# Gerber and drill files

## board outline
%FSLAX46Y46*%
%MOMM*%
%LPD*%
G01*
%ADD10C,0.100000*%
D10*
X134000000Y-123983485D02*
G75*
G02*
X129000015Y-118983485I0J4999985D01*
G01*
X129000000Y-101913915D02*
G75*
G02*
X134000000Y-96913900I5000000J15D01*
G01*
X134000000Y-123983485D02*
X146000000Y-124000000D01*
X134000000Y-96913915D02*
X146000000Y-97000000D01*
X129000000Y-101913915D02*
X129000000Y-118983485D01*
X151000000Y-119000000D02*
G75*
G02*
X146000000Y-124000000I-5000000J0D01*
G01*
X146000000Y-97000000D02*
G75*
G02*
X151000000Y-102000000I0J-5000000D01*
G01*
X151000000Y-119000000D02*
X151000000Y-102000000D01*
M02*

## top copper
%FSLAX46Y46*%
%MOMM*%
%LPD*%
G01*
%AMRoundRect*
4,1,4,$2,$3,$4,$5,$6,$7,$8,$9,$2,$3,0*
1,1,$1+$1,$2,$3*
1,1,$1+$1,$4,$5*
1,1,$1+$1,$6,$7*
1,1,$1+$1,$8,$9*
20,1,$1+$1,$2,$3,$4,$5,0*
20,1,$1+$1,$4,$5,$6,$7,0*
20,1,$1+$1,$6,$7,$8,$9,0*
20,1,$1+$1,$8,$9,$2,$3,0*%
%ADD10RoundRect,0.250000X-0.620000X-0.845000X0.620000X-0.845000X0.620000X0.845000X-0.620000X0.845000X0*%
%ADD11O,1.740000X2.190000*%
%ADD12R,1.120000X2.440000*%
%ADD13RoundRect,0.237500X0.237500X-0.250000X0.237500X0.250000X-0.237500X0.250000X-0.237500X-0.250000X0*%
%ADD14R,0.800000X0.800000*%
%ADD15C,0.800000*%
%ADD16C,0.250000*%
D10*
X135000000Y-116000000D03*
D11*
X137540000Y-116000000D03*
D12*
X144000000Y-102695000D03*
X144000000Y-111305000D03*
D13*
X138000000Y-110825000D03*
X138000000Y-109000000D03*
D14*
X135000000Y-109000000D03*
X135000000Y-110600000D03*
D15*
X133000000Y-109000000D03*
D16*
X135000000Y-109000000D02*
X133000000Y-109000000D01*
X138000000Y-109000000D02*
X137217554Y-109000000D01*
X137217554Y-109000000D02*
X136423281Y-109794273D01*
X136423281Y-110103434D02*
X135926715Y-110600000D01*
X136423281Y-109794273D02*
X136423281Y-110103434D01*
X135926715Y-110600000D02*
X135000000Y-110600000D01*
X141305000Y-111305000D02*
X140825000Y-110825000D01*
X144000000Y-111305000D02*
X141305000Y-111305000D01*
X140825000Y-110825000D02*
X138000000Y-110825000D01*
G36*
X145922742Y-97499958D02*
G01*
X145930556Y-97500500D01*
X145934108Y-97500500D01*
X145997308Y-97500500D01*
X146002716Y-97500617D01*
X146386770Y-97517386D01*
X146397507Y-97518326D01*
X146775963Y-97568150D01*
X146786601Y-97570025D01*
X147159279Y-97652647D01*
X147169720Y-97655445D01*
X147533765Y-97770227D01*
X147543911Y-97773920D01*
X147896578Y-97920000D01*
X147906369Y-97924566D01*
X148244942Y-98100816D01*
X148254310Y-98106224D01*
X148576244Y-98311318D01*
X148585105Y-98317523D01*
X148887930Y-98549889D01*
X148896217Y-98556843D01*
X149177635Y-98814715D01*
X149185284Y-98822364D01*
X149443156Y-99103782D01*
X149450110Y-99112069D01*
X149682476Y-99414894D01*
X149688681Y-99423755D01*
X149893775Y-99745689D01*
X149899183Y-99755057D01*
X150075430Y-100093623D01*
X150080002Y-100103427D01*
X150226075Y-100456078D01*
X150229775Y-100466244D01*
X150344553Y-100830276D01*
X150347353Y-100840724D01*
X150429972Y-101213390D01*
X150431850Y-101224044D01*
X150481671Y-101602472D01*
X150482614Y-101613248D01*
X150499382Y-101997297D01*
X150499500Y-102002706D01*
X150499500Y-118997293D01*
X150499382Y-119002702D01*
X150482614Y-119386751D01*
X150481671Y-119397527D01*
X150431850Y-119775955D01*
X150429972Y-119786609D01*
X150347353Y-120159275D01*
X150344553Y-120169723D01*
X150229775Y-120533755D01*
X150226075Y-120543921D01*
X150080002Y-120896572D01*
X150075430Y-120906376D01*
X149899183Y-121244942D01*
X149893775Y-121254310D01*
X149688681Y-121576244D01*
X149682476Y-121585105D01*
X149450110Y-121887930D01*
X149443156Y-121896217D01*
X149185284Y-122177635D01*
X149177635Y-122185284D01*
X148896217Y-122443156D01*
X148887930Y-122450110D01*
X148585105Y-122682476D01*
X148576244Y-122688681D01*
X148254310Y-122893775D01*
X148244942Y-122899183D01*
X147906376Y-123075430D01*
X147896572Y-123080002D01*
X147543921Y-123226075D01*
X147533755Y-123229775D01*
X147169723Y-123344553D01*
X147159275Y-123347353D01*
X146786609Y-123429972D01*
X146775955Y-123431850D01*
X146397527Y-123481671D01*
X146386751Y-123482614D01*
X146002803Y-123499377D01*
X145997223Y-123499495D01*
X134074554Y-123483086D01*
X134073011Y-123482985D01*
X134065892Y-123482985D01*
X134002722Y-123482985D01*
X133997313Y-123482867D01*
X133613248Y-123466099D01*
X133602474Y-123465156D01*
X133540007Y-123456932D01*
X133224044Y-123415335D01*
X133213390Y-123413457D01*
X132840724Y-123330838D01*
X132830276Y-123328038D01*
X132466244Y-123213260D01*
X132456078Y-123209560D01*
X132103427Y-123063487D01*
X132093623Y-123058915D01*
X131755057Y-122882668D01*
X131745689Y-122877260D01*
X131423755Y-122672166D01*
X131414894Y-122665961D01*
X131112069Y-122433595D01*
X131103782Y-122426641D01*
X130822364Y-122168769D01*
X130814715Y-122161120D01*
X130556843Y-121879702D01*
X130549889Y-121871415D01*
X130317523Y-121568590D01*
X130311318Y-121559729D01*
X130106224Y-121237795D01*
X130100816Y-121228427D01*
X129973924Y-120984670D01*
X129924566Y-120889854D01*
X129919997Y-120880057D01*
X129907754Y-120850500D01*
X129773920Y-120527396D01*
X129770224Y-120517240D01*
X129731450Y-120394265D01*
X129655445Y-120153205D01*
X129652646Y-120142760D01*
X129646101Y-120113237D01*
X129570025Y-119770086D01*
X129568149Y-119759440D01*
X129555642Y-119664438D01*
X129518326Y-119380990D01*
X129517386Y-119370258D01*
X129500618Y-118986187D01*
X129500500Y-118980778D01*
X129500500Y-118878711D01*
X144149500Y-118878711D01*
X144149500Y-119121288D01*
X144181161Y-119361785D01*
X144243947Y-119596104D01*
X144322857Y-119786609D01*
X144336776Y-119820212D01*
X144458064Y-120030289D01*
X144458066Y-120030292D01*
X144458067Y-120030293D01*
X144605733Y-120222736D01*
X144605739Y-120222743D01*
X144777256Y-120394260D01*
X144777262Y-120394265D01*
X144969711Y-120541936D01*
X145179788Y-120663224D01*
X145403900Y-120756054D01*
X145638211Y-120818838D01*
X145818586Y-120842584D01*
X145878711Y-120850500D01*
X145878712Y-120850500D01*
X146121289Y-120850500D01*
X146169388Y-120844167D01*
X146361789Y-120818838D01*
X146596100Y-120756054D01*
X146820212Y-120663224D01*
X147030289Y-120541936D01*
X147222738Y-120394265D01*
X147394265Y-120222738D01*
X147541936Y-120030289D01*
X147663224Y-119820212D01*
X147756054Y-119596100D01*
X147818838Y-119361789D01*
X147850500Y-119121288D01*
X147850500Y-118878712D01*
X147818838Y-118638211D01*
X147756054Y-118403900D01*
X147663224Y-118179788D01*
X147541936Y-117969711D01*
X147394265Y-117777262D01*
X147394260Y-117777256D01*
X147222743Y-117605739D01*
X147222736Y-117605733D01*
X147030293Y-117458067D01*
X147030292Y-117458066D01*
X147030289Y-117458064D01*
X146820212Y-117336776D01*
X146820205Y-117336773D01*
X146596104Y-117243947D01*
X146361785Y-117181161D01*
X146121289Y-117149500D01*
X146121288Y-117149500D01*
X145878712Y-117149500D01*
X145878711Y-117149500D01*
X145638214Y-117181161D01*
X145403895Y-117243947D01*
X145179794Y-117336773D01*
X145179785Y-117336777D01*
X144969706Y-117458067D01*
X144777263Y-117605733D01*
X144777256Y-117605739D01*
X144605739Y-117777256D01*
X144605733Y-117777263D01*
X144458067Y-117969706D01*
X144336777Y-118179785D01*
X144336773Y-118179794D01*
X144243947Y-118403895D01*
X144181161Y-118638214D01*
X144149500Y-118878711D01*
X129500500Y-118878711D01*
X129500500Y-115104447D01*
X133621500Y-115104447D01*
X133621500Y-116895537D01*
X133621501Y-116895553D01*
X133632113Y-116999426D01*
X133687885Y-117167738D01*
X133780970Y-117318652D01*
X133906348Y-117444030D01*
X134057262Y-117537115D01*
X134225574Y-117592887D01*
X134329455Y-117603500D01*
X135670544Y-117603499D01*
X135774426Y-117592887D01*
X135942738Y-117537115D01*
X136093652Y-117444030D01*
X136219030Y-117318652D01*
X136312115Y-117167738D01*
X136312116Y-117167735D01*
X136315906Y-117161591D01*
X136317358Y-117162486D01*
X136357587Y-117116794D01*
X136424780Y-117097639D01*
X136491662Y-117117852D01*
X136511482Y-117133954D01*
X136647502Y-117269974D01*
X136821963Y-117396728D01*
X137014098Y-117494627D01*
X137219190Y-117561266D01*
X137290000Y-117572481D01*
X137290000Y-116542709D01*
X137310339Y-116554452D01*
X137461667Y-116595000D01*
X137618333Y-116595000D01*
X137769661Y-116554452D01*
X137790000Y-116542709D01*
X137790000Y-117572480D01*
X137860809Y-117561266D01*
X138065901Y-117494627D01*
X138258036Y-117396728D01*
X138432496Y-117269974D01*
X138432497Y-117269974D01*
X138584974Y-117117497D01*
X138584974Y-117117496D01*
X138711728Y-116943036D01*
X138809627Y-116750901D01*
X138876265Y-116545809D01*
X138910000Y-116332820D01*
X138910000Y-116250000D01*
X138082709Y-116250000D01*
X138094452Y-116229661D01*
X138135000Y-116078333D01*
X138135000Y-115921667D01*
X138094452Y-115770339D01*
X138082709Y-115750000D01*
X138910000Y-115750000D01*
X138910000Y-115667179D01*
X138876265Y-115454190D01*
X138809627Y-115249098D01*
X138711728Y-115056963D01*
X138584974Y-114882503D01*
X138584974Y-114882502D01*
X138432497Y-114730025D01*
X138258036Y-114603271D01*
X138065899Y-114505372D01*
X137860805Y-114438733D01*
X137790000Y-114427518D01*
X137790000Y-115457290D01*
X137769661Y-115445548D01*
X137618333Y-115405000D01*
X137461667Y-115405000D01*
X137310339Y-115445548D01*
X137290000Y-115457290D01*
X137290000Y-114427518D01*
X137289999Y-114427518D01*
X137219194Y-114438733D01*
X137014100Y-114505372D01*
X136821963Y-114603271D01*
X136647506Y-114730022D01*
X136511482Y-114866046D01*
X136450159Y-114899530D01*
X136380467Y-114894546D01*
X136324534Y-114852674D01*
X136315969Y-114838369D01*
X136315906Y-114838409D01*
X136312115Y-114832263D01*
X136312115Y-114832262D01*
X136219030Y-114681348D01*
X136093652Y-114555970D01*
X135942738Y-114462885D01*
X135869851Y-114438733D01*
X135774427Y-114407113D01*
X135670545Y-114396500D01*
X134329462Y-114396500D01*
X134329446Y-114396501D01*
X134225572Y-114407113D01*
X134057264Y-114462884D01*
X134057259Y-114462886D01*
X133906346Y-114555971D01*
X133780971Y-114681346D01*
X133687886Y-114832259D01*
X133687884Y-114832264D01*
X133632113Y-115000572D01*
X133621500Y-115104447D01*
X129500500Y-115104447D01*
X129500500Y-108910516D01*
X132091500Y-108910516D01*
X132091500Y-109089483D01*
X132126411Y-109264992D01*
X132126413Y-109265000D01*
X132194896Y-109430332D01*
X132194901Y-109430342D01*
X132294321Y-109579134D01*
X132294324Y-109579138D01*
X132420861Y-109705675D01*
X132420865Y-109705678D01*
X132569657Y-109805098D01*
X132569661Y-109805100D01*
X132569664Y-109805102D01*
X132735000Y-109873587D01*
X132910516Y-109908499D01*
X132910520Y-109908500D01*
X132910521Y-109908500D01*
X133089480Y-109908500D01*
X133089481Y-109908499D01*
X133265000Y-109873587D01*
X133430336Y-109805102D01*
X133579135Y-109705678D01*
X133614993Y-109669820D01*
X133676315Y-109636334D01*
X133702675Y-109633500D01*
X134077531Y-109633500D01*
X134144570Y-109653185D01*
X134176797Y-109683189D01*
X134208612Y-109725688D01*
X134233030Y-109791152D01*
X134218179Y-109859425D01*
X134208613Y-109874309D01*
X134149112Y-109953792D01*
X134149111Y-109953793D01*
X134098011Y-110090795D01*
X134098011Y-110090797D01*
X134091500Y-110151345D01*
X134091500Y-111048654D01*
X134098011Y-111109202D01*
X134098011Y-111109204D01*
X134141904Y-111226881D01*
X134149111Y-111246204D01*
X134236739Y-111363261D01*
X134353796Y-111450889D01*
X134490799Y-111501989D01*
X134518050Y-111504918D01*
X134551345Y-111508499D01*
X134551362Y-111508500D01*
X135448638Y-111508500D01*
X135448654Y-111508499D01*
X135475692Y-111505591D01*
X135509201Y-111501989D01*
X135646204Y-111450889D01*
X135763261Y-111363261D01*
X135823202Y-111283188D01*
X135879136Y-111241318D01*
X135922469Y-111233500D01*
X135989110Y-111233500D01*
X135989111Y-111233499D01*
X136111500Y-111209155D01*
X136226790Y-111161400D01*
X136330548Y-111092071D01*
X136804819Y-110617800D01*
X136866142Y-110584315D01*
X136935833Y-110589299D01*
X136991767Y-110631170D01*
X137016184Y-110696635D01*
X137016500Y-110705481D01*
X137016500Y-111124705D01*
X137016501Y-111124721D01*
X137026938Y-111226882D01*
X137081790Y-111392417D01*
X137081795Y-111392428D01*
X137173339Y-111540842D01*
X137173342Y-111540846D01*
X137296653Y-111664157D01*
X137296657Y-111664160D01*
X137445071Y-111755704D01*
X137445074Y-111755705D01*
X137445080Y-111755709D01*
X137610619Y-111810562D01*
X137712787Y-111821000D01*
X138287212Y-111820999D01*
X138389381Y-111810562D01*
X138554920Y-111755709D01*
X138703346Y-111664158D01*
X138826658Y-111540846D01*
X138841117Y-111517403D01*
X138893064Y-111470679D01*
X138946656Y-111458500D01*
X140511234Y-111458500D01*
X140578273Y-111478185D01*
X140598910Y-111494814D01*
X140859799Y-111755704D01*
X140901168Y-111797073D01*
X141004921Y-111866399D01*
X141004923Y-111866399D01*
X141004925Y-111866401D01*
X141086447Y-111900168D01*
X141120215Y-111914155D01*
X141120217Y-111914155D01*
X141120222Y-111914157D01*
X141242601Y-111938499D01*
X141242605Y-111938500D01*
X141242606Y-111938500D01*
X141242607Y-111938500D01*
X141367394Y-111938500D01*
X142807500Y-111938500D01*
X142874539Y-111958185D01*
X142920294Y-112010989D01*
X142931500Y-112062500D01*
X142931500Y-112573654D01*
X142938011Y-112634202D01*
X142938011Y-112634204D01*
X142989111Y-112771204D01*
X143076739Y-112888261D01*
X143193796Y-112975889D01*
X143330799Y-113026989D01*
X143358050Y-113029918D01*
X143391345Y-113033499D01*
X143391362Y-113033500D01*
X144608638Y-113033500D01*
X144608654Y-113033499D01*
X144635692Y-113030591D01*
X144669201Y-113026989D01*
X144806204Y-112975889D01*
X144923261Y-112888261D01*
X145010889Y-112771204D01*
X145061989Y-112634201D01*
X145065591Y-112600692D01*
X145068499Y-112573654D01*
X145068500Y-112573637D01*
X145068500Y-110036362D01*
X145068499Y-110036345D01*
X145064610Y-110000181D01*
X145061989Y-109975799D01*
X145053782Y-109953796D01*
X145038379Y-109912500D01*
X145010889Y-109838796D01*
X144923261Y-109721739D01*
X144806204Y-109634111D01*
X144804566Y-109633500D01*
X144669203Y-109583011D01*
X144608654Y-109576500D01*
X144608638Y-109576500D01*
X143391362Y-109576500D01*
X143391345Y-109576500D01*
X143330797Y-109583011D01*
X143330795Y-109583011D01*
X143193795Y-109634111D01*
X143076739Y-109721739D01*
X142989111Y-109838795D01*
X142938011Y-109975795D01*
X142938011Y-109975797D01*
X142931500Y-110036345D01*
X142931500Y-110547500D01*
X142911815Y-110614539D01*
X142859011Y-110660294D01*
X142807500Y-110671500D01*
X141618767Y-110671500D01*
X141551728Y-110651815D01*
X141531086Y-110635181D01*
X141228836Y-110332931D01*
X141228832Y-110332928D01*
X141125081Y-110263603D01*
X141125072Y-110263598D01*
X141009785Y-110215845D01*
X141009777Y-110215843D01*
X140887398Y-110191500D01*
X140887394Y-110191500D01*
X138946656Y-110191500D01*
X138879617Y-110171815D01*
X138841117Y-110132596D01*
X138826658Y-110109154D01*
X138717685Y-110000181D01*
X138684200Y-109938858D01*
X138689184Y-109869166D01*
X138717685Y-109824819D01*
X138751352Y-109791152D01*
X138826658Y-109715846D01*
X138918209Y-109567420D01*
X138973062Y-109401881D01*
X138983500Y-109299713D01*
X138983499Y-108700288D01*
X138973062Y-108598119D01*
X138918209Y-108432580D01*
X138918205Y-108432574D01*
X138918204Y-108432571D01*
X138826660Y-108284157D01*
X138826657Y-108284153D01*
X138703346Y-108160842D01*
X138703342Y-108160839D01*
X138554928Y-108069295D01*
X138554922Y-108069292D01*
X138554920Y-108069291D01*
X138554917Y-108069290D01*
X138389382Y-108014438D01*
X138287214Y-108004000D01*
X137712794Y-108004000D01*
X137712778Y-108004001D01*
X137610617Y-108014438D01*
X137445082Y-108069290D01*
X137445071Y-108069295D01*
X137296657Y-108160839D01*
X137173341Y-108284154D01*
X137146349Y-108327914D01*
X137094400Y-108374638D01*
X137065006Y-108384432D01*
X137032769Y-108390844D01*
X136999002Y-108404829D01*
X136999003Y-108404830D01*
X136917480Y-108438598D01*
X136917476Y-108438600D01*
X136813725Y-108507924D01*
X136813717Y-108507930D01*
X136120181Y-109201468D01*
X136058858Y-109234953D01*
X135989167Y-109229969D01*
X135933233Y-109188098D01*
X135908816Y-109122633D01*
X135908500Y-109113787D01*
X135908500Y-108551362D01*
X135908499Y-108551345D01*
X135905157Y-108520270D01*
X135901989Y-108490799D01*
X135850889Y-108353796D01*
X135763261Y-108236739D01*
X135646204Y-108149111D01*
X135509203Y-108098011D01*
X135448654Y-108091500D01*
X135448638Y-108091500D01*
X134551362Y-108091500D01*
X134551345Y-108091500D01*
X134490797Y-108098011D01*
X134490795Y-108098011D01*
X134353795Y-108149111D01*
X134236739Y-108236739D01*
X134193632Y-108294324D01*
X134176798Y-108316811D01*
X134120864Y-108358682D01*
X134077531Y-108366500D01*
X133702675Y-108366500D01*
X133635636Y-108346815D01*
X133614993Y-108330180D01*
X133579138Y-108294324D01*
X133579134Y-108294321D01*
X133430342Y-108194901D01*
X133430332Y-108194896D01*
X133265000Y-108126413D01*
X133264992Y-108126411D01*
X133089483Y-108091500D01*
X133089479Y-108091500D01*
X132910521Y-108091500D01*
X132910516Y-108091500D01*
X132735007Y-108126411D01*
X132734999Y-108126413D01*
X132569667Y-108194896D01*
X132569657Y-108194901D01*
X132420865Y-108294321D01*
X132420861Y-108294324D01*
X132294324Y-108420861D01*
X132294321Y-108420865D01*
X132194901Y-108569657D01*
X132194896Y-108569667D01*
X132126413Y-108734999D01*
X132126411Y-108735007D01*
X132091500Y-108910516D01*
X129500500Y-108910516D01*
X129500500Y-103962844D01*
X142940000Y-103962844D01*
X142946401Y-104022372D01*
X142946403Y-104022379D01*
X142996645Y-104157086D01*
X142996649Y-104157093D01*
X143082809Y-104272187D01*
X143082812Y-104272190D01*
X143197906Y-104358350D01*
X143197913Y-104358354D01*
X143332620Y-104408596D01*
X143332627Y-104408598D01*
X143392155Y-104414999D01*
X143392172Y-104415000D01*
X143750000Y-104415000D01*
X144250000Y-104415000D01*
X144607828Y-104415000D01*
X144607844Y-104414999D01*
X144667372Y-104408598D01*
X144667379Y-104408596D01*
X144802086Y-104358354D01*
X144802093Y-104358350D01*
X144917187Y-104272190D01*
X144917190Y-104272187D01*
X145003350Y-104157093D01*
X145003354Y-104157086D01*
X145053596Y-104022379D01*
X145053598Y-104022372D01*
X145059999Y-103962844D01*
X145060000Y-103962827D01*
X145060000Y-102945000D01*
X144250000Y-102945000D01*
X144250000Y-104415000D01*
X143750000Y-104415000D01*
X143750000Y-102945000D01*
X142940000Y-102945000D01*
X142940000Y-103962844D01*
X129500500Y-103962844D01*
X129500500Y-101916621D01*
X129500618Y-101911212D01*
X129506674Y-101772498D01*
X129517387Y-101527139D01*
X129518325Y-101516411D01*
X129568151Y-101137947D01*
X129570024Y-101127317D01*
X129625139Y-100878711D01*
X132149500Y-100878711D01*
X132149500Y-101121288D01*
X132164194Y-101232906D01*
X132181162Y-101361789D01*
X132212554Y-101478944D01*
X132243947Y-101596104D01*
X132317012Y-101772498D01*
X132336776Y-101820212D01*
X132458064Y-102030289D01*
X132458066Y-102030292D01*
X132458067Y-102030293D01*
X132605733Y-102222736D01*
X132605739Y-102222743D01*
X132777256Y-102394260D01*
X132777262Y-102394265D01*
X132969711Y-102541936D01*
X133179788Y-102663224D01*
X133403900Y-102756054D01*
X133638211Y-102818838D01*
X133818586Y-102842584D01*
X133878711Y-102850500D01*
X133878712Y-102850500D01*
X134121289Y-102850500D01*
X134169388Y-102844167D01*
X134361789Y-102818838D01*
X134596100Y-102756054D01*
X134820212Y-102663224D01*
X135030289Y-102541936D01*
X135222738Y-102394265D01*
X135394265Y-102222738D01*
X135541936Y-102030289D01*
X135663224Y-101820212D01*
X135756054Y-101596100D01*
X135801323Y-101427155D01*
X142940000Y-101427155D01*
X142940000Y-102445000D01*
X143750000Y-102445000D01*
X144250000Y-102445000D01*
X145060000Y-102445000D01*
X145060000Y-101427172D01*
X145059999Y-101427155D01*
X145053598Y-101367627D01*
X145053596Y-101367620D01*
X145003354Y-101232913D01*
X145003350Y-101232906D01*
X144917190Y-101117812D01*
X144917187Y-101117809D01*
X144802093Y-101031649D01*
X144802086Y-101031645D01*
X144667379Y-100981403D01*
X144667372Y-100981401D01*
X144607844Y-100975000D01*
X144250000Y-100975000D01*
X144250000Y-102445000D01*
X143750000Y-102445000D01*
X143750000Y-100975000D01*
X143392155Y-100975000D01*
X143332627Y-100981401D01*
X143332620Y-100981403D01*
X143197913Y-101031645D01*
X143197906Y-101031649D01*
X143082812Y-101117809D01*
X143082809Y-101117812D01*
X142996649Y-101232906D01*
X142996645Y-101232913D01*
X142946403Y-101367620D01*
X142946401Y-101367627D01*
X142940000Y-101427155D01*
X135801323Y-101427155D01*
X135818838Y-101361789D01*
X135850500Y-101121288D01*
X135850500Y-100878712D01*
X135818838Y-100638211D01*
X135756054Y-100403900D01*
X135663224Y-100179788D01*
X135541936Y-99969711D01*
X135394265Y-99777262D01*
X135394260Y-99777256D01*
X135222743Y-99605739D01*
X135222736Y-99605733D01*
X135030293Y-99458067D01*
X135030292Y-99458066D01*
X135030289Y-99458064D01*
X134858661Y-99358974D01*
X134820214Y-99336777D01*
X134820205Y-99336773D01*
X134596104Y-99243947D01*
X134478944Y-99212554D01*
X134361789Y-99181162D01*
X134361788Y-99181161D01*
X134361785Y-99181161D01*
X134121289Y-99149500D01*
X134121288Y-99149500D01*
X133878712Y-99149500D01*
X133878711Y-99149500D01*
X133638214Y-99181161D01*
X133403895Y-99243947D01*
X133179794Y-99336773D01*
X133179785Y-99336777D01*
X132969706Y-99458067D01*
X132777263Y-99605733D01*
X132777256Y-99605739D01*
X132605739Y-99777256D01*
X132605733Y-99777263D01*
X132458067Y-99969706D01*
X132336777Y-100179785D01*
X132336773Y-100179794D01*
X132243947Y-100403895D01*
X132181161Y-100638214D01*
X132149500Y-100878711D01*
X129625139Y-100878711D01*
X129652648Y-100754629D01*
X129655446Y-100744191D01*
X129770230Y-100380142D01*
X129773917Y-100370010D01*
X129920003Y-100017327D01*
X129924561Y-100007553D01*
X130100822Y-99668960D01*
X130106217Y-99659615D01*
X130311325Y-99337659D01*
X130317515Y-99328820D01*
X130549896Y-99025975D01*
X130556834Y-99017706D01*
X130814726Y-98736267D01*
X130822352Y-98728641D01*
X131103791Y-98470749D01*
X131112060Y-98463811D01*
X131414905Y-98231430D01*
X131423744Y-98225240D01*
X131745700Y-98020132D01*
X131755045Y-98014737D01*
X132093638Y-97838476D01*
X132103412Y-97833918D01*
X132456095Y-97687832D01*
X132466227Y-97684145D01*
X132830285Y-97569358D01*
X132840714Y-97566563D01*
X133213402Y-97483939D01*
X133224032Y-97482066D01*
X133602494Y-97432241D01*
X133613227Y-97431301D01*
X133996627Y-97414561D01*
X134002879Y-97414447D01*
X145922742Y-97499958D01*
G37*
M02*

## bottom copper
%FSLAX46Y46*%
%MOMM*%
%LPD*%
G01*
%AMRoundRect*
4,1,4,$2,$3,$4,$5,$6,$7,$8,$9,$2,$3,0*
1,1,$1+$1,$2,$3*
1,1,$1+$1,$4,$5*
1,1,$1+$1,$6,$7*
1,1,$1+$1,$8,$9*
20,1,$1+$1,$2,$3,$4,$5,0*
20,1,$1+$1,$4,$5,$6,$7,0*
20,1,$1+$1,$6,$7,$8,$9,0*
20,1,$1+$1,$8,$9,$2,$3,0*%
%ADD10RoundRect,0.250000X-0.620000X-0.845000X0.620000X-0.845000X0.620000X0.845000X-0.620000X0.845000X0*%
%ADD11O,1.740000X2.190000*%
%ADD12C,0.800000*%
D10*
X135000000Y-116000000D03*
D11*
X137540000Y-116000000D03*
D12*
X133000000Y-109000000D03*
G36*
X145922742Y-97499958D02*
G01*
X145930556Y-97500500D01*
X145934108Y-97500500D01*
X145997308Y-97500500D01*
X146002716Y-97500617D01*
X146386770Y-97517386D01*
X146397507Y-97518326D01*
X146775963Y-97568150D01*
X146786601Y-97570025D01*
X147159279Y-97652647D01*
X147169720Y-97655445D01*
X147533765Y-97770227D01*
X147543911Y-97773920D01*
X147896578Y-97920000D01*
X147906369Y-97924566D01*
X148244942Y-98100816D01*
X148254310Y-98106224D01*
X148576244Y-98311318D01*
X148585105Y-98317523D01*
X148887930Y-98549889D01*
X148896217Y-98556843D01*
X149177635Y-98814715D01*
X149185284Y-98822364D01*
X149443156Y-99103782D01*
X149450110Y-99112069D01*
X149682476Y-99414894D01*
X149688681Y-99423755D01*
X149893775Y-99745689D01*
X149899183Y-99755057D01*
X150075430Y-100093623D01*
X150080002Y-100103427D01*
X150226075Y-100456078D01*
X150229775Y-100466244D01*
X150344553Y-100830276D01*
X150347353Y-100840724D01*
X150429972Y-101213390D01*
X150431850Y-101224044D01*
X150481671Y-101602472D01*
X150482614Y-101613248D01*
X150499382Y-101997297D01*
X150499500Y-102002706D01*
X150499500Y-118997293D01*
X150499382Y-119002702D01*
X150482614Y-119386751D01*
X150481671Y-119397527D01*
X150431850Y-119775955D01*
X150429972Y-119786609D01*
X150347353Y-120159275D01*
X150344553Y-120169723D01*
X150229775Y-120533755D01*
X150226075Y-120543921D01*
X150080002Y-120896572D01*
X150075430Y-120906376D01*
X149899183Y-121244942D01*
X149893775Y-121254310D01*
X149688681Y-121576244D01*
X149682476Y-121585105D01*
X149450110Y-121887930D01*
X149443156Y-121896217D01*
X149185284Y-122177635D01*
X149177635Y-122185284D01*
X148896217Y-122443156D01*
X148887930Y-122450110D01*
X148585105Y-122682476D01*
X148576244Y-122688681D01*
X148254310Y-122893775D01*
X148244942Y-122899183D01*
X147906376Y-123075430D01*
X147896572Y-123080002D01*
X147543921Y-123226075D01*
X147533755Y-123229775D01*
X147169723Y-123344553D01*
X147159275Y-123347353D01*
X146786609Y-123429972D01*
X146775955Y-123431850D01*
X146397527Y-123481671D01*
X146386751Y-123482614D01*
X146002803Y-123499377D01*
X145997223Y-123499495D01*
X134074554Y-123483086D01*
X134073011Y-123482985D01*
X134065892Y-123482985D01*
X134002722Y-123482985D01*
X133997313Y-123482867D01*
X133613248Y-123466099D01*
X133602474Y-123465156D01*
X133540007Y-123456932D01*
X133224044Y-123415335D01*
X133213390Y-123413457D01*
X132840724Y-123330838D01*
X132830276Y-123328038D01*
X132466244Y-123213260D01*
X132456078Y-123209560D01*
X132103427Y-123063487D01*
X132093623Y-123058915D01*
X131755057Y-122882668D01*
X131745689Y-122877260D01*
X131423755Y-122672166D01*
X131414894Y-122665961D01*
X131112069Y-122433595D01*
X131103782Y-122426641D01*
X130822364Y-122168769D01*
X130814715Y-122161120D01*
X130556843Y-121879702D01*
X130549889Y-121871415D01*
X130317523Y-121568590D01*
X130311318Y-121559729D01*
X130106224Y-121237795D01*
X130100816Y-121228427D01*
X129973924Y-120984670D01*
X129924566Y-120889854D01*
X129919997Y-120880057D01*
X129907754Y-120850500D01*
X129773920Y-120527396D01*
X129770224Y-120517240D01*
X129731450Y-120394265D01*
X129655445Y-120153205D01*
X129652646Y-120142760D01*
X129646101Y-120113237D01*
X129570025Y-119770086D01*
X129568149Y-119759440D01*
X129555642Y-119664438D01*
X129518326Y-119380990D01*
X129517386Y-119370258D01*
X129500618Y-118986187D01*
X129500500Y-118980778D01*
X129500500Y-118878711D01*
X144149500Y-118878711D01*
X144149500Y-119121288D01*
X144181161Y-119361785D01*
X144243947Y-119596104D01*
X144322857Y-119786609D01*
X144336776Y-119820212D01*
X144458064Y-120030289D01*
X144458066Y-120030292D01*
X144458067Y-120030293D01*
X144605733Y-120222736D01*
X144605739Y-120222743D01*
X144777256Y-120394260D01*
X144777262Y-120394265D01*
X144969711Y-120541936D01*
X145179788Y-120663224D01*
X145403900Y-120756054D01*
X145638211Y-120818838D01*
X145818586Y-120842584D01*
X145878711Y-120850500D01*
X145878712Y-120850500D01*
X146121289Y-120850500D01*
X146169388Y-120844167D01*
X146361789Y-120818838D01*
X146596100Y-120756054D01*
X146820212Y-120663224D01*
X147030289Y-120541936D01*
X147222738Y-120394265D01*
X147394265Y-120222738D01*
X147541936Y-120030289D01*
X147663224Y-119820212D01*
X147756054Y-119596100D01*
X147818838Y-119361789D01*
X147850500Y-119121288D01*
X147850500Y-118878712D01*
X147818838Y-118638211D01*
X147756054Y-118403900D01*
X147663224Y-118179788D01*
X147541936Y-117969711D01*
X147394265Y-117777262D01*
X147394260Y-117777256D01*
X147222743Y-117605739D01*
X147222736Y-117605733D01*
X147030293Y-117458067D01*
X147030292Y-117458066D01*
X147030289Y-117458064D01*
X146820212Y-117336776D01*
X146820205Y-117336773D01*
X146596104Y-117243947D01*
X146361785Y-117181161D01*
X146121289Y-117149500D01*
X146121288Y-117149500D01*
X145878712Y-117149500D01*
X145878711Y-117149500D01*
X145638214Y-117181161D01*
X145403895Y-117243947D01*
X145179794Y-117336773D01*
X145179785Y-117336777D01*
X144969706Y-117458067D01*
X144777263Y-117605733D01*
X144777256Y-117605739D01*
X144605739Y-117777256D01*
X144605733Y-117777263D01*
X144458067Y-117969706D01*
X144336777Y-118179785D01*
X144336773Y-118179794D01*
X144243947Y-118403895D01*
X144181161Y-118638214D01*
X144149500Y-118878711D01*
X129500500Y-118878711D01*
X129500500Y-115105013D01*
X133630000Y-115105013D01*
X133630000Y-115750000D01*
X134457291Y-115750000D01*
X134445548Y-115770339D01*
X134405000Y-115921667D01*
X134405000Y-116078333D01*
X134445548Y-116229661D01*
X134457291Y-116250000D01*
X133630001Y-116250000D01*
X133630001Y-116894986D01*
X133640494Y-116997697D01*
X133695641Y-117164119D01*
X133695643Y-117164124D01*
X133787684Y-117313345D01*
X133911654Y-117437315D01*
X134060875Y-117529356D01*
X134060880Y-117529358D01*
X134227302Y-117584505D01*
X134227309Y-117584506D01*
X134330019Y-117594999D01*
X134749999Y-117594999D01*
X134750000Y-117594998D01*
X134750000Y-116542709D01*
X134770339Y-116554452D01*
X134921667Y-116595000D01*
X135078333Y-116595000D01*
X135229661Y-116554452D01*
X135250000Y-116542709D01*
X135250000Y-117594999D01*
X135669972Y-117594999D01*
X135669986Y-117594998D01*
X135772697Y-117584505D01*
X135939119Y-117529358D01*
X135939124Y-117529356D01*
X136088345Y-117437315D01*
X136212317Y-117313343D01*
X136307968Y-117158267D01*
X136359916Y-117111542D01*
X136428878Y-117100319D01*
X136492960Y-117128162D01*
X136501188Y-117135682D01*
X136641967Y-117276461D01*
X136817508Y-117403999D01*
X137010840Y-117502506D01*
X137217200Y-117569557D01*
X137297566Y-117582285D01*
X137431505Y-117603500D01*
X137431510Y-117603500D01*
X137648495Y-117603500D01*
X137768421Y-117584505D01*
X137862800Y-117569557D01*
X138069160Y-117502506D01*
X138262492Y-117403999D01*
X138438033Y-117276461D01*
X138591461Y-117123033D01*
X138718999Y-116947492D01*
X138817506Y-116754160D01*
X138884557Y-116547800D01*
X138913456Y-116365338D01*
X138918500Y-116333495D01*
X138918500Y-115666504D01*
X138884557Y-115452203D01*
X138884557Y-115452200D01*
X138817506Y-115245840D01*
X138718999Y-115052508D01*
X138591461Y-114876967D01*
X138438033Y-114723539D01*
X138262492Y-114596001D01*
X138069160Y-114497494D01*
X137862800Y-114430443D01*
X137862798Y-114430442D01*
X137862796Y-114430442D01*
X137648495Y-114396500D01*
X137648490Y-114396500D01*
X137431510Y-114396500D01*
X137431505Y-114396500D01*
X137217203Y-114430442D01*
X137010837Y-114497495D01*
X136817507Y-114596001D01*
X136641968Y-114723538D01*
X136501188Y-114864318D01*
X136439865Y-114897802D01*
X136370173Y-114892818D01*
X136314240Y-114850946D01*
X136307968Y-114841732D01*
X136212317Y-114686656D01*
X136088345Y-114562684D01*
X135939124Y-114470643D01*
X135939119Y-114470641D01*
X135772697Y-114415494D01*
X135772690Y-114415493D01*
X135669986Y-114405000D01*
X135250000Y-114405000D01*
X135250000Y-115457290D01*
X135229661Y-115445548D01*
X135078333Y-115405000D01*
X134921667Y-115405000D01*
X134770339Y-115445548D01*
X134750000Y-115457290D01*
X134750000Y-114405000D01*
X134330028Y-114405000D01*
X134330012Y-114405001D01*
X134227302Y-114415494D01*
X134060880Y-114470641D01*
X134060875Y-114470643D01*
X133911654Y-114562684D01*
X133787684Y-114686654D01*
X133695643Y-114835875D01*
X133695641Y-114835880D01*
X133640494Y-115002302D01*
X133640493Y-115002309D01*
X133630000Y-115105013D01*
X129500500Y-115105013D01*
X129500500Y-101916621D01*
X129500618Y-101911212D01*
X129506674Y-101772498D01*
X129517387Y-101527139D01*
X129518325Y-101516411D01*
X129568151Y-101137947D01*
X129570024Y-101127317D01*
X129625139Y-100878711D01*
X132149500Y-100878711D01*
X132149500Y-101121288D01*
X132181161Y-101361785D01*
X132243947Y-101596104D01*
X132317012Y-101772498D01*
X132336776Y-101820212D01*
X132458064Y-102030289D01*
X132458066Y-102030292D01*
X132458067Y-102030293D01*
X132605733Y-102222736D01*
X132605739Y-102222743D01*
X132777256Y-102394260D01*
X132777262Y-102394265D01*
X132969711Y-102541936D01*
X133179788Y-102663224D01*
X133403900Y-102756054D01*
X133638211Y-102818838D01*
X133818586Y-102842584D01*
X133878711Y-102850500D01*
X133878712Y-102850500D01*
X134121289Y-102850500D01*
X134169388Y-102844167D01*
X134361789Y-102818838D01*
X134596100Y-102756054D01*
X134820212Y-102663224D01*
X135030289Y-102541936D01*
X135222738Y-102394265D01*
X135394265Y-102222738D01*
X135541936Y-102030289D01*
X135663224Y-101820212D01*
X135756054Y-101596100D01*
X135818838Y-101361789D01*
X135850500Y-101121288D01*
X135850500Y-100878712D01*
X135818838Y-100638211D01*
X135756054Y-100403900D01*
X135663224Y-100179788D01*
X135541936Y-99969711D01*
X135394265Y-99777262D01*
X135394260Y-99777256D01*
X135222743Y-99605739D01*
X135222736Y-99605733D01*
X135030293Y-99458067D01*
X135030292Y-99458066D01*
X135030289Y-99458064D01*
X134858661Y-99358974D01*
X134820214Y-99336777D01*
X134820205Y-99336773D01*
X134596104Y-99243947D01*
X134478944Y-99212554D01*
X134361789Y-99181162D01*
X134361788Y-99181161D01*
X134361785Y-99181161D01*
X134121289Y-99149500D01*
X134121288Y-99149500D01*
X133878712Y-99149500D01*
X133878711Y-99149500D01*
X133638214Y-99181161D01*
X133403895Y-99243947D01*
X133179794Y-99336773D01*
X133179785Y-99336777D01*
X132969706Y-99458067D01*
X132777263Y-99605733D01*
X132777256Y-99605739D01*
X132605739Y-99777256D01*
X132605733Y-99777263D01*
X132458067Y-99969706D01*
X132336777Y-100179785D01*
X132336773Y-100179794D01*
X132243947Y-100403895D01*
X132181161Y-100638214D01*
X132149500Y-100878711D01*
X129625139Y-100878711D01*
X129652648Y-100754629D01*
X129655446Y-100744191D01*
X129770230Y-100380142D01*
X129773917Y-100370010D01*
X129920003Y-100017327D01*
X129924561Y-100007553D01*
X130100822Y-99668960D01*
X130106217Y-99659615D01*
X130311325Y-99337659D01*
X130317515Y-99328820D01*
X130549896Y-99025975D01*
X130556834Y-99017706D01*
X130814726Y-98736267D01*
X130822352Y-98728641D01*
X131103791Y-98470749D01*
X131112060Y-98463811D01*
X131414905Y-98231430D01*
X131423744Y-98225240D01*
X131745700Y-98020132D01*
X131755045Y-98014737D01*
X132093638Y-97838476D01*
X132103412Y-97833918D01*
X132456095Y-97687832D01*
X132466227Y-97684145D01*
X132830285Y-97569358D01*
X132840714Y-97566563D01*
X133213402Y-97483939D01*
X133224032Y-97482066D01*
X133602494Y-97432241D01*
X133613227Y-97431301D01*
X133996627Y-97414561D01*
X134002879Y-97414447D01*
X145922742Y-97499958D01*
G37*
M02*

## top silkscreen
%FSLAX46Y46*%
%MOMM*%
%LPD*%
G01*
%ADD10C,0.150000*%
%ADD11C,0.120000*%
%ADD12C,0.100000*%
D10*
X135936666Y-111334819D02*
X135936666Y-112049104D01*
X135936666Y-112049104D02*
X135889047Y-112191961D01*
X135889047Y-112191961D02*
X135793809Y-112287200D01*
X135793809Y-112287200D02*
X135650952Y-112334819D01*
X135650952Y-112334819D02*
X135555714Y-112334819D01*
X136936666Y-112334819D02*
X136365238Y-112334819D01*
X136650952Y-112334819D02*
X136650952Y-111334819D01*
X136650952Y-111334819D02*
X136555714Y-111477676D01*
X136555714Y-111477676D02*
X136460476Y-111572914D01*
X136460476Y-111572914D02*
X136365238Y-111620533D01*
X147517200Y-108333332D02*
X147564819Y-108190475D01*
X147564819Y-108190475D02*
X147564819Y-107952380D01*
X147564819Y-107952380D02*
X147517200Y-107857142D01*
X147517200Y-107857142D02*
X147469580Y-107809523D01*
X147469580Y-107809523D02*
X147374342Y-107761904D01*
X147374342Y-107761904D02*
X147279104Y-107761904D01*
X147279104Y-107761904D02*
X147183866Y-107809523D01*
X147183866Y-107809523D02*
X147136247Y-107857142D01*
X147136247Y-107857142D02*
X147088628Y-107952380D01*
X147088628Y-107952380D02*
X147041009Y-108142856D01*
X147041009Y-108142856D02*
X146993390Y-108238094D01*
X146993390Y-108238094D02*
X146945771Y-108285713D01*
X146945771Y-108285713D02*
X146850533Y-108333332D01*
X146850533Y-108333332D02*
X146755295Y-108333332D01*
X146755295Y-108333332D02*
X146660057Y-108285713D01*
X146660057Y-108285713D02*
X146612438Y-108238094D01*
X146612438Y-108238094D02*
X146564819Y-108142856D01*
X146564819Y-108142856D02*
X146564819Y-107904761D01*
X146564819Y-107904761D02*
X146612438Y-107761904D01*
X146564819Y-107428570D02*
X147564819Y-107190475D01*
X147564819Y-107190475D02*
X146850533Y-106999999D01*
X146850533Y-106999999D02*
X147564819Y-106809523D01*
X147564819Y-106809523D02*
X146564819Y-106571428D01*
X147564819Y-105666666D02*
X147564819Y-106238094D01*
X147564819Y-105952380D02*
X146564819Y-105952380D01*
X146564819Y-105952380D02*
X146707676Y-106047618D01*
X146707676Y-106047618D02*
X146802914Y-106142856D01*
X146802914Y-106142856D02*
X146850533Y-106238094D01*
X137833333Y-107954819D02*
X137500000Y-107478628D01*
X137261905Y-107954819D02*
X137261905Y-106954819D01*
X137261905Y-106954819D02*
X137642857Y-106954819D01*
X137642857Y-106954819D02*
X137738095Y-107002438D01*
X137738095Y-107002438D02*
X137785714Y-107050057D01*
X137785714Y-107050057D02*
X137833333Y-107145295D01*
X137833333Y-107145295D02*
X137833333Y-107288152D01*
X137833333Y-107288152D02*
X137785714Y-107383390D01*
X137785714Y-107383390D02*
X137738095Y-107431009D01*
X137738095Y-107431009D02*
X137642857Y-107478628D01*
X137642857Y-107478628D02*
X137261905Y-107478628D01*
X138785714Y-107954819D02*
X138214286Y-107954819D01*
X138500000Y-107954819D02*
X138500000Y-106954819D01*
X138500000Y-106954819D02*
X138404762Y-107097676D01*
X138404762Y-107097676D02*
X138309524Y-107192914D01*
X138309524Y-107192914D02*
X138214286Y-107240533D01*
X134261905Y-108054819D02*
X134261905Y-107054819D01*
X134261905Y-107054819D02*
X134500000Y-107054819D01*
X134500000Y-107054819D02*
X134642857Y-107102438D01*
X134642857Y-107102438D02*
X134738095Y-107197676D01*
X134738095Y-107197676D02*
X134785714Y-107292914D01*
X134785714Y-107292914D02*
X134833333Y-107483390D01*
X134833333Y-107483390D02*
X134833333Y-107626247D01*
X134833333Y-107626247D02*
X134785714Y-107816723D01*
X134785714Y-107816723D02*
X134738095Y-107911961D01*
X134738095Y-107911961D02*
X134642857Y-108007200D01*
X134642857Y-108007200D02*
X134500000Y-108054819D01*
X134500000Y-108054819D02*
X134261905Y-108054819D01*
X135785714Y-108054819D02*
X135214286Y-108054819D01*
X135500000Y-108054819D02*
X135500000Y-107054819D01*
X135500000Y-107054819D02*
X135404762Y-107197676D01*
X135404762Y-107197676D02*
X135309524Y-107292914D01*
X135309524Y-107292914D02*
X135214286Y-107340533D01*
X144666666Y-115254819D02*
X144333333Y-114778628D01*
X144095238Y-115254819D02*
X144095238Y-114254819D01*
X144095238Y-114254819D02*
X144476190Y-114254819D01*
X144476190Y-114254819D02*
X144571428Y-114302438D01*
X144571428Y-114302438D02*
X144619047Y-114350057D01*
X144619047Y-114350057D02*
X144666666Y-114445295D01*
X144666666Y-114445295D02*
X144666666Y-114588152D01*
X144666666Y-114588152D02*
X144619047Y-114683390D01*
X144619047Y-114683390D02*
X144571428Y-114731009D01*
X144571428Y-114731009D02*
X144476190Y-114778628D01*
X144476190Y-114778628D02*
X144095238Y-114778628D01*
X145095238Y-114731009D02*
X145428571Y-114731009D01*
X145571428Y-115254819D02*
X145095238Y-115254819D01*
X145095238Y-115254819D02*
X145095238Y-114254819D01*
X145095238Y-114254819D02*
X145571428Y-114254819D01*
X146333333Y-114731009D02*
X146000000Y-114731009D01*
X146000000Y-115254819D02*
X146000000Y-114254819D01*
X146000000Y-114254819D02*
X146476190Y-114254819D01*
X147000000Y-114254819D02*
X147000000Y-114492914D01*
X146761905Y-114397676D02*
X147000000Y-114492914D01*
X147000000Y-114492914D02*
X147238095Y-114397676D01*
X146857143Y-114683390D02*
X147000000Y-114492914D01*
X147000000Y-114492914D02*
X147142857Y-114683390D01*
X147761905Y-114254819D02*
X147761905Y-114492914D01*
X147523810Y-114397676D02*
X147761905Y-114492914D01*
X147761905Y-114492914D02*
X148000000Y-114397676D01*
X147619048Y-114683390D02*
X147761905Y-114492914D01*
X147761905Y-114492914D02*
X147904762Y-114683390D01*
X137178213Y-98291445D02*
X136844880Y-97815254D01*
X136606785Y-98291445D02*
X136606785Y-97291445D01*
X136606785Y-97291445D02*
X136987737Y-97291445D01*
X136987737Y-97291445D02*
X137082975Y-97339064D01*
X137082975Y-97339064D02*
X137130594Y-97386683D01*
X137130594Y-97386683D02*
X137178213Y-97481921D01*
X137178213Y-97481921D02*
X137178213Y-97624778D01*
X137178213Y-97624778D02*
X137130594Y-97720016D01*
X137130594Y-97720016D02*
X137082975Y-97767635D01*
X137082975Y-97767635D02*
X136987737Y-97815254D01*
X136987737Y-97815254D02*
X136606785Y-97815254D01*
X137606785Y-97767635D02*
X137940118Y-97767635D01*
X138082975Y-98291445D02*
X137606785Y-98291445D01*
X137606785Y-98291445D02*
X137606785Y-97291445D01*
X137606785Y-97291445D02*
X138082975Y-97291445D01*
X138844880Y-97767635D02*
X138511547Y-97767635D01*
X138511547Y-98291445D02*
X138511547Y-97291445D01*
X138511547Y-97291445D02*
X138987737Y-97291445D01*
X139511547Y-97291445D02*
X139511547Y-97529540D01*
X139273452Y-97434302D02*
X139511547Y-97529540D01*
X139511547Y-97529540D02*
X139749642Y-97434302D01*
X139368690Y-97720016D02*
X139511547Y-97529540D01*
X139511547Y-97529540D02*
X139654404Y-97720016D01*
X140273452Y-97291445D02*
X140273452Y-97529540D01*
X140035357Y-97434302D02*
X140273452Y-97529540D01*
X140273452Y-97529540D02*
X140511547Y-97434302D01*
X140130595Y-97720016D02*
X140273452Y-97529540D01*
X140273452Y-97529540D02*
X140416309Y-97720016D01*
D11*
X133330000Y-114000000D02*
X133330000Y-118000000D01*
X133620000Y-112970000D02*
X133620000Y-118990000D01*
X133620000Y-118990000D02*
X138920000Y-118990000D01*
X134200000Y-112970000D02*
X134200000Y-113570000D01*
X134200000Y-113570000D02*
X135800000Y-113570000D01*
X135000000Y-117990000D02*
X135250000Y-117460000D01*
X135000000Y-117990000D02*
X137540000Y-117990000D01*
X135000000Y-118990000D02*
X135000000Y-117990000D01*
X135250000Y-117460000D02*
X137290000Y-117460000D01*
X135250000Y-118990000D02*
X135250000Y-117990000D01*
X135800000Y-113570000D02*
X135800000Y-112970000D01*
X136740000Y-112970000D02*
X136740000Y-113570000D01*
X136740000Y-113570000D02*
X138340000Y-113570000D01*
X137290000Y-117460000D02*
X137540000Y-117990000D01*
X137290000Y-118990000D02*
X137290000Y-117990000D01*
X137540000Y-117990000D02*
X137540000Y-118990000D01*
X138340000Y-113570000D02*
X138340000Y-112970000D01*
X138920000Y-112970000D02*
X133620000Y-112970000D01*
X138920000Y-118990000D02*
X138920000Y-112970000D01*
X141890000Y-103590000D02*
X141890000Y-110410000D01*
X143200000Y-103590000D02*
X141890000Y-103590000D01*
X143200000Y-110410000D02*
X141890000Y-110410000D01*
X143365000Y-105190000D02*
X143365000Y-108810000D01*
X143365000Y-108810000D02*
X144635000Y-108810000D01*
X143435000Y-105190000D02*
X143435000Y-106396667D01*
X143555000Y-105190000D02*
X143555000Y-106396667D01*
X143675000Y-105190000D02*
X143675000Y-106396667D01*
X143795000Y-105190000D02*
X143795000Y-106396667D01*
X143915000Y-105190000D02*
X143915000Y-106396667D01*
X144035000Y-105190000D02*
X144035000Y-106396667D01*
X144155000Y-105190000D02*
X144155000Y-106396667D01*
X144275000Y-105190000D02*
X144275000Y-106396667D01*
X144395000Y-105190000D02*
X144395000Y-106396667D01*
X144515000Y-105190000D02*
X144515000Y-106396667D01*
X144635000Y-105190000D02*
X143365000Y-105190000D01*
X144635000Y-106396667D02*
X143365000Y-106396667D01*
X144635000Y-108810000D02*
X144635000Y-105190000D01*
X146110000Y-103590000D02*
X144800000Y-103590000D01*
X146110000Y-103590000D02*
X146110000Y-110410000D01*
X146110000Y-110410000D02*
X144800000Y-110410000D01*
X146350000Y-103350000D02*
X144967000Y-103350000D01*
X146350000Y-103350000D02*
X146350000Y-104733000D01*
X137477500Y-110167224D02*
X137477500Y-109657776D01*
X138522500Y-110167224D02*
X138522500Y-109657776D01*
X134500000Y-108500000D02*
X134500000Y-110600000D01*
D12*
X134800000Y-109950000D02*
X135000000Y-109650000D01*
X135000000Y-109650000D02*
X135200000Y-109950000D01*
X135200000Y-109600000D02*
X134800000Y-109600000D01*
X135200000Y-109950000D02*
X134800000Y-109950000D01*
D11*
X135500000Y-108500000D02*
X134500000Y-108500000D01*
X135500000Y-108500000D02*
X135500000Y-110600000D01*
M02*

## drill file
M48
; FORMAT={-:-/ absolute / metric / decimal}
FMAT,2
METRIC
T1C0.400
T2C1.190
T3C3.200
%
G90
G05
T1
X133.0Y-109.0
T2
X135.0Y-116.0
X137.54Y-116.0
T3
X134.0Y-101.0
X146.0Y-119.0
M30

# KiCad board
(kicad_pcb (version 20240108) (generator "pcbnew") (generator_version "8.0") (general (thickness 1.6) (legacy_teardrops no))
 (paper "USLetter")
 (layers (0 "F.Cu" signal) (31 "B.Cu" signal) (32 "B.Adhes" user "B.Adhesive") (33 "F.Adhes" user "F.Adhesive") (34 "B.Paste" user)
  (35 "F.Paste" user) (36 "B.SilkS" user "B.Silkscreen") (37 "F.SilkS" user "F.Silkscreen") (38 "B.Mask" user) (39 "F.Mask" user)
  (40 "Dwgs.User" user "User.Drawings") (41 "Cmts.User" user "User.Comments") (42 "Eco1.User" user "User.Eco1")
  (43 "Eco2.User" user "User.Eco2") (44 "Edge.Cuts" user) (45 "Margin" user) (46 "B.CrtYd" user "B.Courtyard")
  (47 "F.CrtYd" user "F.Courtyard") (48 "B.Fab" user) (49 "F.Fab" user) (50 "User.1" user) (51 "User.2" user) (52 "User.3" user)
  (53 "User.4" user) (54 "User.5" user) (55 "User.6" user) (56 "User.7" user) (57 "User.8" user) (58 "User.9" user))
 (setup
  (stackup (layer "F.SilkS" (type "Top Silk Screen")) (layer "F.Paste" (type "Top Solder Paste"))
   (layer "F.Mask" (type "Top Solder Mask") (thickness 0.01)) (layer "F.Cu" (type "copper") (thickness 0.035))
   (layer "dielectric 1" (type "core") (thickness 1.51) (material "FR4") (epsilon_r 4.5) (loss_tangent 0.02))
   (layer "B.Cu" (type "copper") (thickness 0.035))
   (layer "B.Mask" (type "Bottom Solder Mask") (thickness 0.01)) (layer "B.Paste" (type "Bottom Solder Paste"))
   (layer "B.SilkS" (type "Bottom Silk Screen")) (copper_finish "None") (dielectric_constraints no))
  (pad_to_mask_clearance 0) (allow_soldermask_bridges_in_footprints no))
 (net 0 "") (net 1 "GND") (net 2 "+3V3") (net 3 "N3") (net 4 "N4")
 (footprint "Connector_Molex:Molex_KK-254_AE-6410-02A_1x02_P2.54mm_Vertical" (layer "F.Cu") (at 135 116)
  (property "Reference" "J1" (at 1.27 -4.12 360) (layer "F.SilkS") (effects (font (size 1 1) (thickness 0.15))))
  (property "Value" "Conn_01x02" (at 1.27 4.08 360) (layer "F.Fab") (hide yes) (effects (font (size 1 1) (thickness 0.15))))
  (fp_line (start -1.67 -2) (end -1.67 2) (stroke (width 0.12) (type solid)) (layer "F.SilkS"))
  (fp_line (start -1.38 -3.03) (end -1.38 2.99) (stroke (width 0.12) (type solid)) (layer "F.SilkS"))
  (fp_line (start -1.38 2.99) (end 3.92 2.99) (stroke (width 0.12) (type solid)) (layer "F.SilkS"))
  (fp_line (start -0.8 -3.03) (end -0.8 -2.43) (stroke (width 0.12) (type solid)) (layer "F.SilkS"))
  (fp_line (start -0.8 -2.43) (end 0.8 -2.43) (stroke (width 0.12) (type solid)) (layer "F.SilkS"))
  (fp_line (start 0 1.99) (end 0.25 1.46) (stroke (width 0.12) (type solid)) (layer "F.SilkS"))
  (fp_line (start 0 1.99) (end 2.54 1.99) (stroke (width 0.12) (type solid)) (layer "F.SilkS"))
  (fp_line (start 0 2.99) (end 0 1.99) (stroke (width 0.12) (type solid)) (layer "F.SilkS"))
  (fp_line (start 0.25 1.46) (end 2.29 1.46) (stroke (width 0.12) (type solid)) (layer "F.SilkS"))
  (fp_line (start 0.25 2.99) (end 0.25 1.99) (stroke (width 0.12) (type solid)) (layer "F.SilkS"))
  (fp_line (start 0.8 -2.43) (end 0.8 -3.03) (stroke (width 0.12) (type solid)) (layer "F.SilkS"))
  (fp_line (start 1.74 -3.03) (end 1.74 -2.43) (stroke (width 0.12) (type solid)) (layer "F.SilkS"))
  (fp_line (start 1.74 -2.43) (end 3.34 -2.43) (stroke (width 0.12) (type solid)) (layer "F.SilkS"))
  (fp_line (start 2.29 1.46) (end 2.54 1.99) (stroke (width 0.12) (type solid)) (layer "F.SilkS"))
  (fp_line (start 2.29 2.99) (end 2.29 1.99) (stroke (width 0.12) (type solid)) (layer "F.SilkS"))
  (fp_line (start 2.54 1.99) (end 2.54 2.99) (stroke (width 0.12) (type solid)) (layer "F.SilkS"))
  (fp_line (start 3.34 -2.43) (end 3.34 -3.03) (stroke (width 0.12) (type solid)) (layer "F.SilkS"))
  (fp_line (start 3.92 -3.03) (end -1.38 -3.03) (stroke (width 0.12) (type solid)) (layer "F.SilkS"))
  (fp_line (start 3.92 2.99) (end 3.92 -3.03) (stroke (width 0.12) (type solid)) (layer "F.SilkS"))
  (pad "1" thru_hole roundrect (at 0 0) (size 1.74 2.19) (drill 1.19) (layers "*.Cu" "*.Mask") (remove_unused_layers no)
   (roundrect_rratio 0.143678) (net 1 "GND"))
  (pad "2" thru_hole oval (at 2.54 0) (size 1.74 2.19) (drill 1.19) (layers "*.Cu" "*.Mask") (remove_unused_layers no) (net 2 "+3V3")))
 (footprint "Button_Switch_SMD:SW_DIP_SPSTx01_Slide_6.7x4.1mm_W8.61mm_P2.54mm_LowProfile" (layer "F.Cu") (at 144 107 -90)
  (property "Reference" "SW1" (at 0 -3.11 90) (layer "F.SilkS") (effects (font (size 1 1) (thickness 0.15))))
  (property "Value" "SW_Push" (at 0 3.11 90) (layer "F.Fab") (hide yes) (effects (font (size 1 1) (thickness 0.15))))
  (fp_line (start -3.41 2.11) (end 3.41 2.11) (stroke (width 0.12) (type solid)) (layer "F.SilkS"))
  (fp_line (start -3.41 0.8) (end -3.41 2.11) (stroke (width 0.12) (type solid)) (layer "F.SilkS"))
  (fp_line (start 3.41 0.8) (end 3.41 2.11) (stroke (width 0.12) (type solid)) (layer "F.SilkS"))
  (fp_line (start -1.81 0.635) (end 1.81 0.635) (stroke (width 0.12) (type solid)) (layer "F.SilkS"))
  (fp_line (start 1.81 0.635) (end 1.81 -0.635) (stroke (width 0.12) (type solid)) (layer "F.SilkS"))
  (fp_line (start -1.81 0.565) (end -0.603333 0.565) (stroke (width 0.12) (type solid)) (layer "F.SilkS"))
  (fp_line (start -1.81 0.445) (end -0.603333 0.445) (stroke (width 0.12) (type solid)) (layer "F.SilkS"))
  (fp_line (start -1.81 0.325) (end -0.603333 0.325) (stroke (width 0.12) (type solid)) (layer "F.SilkS"))
  (fp_line (start -1.81 0.205) (end -0.603333 0.205) (stroke (width 0.12) (type solid)) (layer "F.SilkS"))
  (fp_line (start -1.81 0.085) (end -0.603333 0.085) (stroke (width 0.12) (type solid)) (layer "F.SilkS"))
  (fp_line (start -1.81 -0.035) (end -0.603333 -0.035) (stroke (width 0.12) (type solid)) (layer "F.SilkS"))
  (fp_line (start -1.81 -0.155) (end -0.603333 -0.155) (stroke (width 0.12) (type solid)) (layer "F.SilkS"))
  (fp_line (start -1.81 -0.275) (end -0.603333 -0.275) (stroke (width 0.12) (type solid)) (layer "F.SilkS"))
  (fp_line (start -1.81 -0.395) (end -0.603333 -0.395) (stroke (width 0.12) (type solid)) (layer "F.SilkS"))
  (fp_line (start -1.81 -0.515) (end -0.603333 -0.515) (stroke (width 0.12) (type solid)) (layer "F.SilkS"))
  (fp_line (start -1.81 -0.635) (end -1.81 0.635) (stroke (width 0.12) (type solid)) (layer "F.SilkS"))
  (fp_line (start -0.603333 -0.635) (end -0.603333 0.635) (stroke (width 0.12) (type solid)) (layer "F.SilkS"))
  (fp_line (start 1.81 -0.635) (end -1.81 -0.635) (stroke (width 0.12) (type solid)) (layer "F.SilkS"))
  (fp_line (start -3.41 -2.11) (end -3.41 -0.8) (stroke (width 0.12) (type solid)) (layer "F.SilkS"))
  (fp_line (start -3.41 -2.11) (end 3.41 -2.11) (stroke (width 0.12) (type solid)) (layer "F.SilkS"))
  (fp_line (start 3.41 -2.11) (end 3.41 -0.8) (stroke (width 0.12) (type solid)) (layer "F.SilkS"))
  (fp_line (start -3.65 -2.35) (end -3.65 -0.967) (stroke (width 0.12) (type solid)) (layer "F.SilkS"))
  (fp_line (start -3.65 -2.35) (end -2.267 -2.35) (stroke (width 0.12) (type solid)) (layer "F.SilkS"))
  (pad "1" smd rect (at -4.305 0 270) (size 2.44 1.12) (layers "F.Cu" "F.Paste" "F.Mask") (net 2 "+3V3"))
  (pad "2" smd rect (at 4.305 0 270) (size 2.44 1.12) (layers "F.Cu" "F.Paste" "F.Mask") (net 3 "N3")))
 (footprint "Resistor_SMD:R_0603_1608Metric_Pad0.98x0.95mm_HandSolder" (layer "F.Cu") (at 138 109.9125 90)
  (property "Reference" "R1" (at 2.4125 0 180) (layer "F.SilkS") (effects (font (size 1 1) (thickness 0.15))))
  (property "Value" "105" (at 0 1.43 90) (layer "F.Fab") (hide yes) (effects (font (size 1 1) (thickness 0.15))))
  (fp_line (start -0.254724 -0.5225) (end 0.254724 -0.5225) (stroke (width 0.12) (type solid)) (layer "F.SilkS"))
  (fp_line (start -0.254724 0.5225) (end 0.254724 0.5225) (stroke (width 0.12) (type solid)) (layer "F.SilkS"))
  (pad "1" smd roundrect (at -0.9125 0 90) (size 0.975 0.95) (layers "F.Cu" "F.Paste" "F.Mask") (roundrect_rratio 0.25) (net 3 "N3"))
  (pad "2" smd roundrect (at 0.9125 0 90) (size 0.975 0.95) (layers "F.Cu" "F.Paste" "F.Mask") (roundrect_rratio 0.25) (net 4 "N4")))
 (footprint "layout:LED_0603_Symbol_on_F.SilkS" (layer "F.Cu") (at 135 109.8 -90)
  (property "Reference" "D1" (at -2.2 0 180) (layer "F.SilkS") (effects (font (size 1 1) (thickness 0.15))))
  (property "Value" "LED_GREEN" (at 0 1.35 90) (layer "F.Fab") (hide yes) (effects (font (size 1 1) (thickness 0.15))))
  (fp_line (start -1.3 0.5) (end 0.8 0.5) (stroke (width 0.12) (type solid)) (layer "F.SilkS"))
  (fp_line (start 0.15 0.2) (end -0.15 0) (stroke (width 0.1) (type solid)) (layer "F.SilkS"))
  (fp_line (start -0.15 0) (end 0.15 -0.2) (stroke (width 0.1) (type solid)) (layer "F.SilkS"))
  (fp_line (start -0.2 -0.2) (end -0.2 0.2) (stroke (width 0.1) (type solid)) (layer "F.SilkS"))
  (fp_line (start 0.15 -0.2) (end 0.15 0.2) (stroke (width 0.1) (type solid)) (layer "F.SilkS"))
  (fp_line (start -1.3 -0.5) (end -1.3 0.5) (stroke (width 0.12) (type solid)) (layer "F.SilkS"))
  (fp_line (start -1.3 -0.5) (end 0.8 -0.5) (stroke (width 0.12) (type solid)) (layer "F.SilkS"))
  (pad "1" smd rect (at -0.8 0 90) (size 0.8 0.8) (layers "F.Cu" "F.Paste" "F.Mask") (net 1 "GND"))
  (pad "2" smd rect (at 0.8 0 90) (size 0.8 0.8) (layers "F.Cu" "F.Paste" "F.Mask") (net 4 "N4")))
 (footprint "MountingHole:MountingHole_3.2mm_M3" (layer "F.Cu") (at 146 119)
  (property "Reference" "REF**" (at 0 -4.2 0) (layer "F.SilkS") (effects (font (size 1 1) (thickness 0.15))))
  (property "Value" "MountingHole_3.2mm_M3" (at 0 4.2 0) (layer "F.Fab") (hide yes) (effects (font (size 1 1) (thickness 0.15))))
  (pad "" np_thru_hole circle (at 0 0) (size 3.2 3.2) (drill 3.2) (layers "*.Cu" "*.Mask")))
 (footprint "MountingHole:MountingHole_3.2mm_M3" (layer "F.Cu") (at 134 101)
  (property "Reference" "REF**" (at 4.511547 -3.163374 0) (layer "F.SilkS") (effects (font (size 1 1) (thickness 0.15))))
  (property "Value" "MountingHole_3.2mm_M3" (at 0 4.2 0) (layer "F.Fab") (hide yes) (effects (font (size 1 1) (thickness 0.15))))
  (pad "" np_thru_hole circle (at 0 0) (size 3.2 3.2) (drill 3.2) (layers "*.Cu" "*.Mask")))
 (gr_arc (start 134 123.983485) (mid 130.464466 122.519019) (end 129 118.983485) (stroke (width 0.1) (type default)) (layer "Edge.Cuts"))
 (gr_arc (start 129 101.913915) (mid 130.464466 98.378381) (end 134 96.913915) (stroke (width 0.1) (type default)) (layer "Edge.Cuts"))
 (gr_line (start 134 123.983485) (end 146 124) (stroke (width 0.1) (type default)) (layer "Edge.Cuts"))
 (gr_line (start 134 96.913915) (end 146 97) (stroke (width 0.1) (type default)) (layer "Edge.Cuts"))
 (gr_line (start 129 101.913915) (end 129 118.983485) (stroke (width 0.1) (type default)) (layer "Edge.Cuts"))
 (gr_arc (start 151 119) (mid 149.535534 122.535534) (end 146 124) (stroke (width 0.1) (type default)) (layer "Edge.Cuts"))
 (gr_arc (start 146 97) (mid 149.535534 98.464466) (end 151 102) (stroke (width 0.1) (type default)) (layer "Edge.Cuts"))
 (gr_line (start 151 119) (end 151 102) (stroke (width 0.1) (type default)) (layer "Edge.Cuts"))
 (segment (start 135 109) (end 133 109) (width 0.25) (layer "F.Cu") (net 1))
 (via (at 133 109) (size 0.8) (drill 0.4) (layers "F.Cu" "B.Cu") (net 1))
 (segment (start 138 109) (end 137.217554 109) (width 0.25) (layer "F.Cu") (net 4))
 (segment (start 137.217554 109) (end 136.423281 109.794273) (width 0.25) (layer "F.Cu") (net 4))
 (segment (start 136.423281 110.103434) (end 135.926715 110.6) (width 0.25) (layer "F.Cu") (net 4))
 (segment (start 136.423281 109.794273) (end 136.423281 110.103434) (width 0.25) (layer "F.Cu") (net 4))
 (segment (start 135.926715 110.6) (end 135 110.6) (width 0.25) (layer "F.Cu") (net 4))
 (segment (start 141.305 111.305) (end 140.825 110.825) (width 0.25) (layer "F.Cu") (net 3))
 (segment (start 144 111.305) (end 141.305 111.305) (width 0.25) (layer "F.Cu") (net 3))
 (segment (start 140.825 110.825) (end 138 110.825) (width 0.25) (layer "F.Cu") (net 3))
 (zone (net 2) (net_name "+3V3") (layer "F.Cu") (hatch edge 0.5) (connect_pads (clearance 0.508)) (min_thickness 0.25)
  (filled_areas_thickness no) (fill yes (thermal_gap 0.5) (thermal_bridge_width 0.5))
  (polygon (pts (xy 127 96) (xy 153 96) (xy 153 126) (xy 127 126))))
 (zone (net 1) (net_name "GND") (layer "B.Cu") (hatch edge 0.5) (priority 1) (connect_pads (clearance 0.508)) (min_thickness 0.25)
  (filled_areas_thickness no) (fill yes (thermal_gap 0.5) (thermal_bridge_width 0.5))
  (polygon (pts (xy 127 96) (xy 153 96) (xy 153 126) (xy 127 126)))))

